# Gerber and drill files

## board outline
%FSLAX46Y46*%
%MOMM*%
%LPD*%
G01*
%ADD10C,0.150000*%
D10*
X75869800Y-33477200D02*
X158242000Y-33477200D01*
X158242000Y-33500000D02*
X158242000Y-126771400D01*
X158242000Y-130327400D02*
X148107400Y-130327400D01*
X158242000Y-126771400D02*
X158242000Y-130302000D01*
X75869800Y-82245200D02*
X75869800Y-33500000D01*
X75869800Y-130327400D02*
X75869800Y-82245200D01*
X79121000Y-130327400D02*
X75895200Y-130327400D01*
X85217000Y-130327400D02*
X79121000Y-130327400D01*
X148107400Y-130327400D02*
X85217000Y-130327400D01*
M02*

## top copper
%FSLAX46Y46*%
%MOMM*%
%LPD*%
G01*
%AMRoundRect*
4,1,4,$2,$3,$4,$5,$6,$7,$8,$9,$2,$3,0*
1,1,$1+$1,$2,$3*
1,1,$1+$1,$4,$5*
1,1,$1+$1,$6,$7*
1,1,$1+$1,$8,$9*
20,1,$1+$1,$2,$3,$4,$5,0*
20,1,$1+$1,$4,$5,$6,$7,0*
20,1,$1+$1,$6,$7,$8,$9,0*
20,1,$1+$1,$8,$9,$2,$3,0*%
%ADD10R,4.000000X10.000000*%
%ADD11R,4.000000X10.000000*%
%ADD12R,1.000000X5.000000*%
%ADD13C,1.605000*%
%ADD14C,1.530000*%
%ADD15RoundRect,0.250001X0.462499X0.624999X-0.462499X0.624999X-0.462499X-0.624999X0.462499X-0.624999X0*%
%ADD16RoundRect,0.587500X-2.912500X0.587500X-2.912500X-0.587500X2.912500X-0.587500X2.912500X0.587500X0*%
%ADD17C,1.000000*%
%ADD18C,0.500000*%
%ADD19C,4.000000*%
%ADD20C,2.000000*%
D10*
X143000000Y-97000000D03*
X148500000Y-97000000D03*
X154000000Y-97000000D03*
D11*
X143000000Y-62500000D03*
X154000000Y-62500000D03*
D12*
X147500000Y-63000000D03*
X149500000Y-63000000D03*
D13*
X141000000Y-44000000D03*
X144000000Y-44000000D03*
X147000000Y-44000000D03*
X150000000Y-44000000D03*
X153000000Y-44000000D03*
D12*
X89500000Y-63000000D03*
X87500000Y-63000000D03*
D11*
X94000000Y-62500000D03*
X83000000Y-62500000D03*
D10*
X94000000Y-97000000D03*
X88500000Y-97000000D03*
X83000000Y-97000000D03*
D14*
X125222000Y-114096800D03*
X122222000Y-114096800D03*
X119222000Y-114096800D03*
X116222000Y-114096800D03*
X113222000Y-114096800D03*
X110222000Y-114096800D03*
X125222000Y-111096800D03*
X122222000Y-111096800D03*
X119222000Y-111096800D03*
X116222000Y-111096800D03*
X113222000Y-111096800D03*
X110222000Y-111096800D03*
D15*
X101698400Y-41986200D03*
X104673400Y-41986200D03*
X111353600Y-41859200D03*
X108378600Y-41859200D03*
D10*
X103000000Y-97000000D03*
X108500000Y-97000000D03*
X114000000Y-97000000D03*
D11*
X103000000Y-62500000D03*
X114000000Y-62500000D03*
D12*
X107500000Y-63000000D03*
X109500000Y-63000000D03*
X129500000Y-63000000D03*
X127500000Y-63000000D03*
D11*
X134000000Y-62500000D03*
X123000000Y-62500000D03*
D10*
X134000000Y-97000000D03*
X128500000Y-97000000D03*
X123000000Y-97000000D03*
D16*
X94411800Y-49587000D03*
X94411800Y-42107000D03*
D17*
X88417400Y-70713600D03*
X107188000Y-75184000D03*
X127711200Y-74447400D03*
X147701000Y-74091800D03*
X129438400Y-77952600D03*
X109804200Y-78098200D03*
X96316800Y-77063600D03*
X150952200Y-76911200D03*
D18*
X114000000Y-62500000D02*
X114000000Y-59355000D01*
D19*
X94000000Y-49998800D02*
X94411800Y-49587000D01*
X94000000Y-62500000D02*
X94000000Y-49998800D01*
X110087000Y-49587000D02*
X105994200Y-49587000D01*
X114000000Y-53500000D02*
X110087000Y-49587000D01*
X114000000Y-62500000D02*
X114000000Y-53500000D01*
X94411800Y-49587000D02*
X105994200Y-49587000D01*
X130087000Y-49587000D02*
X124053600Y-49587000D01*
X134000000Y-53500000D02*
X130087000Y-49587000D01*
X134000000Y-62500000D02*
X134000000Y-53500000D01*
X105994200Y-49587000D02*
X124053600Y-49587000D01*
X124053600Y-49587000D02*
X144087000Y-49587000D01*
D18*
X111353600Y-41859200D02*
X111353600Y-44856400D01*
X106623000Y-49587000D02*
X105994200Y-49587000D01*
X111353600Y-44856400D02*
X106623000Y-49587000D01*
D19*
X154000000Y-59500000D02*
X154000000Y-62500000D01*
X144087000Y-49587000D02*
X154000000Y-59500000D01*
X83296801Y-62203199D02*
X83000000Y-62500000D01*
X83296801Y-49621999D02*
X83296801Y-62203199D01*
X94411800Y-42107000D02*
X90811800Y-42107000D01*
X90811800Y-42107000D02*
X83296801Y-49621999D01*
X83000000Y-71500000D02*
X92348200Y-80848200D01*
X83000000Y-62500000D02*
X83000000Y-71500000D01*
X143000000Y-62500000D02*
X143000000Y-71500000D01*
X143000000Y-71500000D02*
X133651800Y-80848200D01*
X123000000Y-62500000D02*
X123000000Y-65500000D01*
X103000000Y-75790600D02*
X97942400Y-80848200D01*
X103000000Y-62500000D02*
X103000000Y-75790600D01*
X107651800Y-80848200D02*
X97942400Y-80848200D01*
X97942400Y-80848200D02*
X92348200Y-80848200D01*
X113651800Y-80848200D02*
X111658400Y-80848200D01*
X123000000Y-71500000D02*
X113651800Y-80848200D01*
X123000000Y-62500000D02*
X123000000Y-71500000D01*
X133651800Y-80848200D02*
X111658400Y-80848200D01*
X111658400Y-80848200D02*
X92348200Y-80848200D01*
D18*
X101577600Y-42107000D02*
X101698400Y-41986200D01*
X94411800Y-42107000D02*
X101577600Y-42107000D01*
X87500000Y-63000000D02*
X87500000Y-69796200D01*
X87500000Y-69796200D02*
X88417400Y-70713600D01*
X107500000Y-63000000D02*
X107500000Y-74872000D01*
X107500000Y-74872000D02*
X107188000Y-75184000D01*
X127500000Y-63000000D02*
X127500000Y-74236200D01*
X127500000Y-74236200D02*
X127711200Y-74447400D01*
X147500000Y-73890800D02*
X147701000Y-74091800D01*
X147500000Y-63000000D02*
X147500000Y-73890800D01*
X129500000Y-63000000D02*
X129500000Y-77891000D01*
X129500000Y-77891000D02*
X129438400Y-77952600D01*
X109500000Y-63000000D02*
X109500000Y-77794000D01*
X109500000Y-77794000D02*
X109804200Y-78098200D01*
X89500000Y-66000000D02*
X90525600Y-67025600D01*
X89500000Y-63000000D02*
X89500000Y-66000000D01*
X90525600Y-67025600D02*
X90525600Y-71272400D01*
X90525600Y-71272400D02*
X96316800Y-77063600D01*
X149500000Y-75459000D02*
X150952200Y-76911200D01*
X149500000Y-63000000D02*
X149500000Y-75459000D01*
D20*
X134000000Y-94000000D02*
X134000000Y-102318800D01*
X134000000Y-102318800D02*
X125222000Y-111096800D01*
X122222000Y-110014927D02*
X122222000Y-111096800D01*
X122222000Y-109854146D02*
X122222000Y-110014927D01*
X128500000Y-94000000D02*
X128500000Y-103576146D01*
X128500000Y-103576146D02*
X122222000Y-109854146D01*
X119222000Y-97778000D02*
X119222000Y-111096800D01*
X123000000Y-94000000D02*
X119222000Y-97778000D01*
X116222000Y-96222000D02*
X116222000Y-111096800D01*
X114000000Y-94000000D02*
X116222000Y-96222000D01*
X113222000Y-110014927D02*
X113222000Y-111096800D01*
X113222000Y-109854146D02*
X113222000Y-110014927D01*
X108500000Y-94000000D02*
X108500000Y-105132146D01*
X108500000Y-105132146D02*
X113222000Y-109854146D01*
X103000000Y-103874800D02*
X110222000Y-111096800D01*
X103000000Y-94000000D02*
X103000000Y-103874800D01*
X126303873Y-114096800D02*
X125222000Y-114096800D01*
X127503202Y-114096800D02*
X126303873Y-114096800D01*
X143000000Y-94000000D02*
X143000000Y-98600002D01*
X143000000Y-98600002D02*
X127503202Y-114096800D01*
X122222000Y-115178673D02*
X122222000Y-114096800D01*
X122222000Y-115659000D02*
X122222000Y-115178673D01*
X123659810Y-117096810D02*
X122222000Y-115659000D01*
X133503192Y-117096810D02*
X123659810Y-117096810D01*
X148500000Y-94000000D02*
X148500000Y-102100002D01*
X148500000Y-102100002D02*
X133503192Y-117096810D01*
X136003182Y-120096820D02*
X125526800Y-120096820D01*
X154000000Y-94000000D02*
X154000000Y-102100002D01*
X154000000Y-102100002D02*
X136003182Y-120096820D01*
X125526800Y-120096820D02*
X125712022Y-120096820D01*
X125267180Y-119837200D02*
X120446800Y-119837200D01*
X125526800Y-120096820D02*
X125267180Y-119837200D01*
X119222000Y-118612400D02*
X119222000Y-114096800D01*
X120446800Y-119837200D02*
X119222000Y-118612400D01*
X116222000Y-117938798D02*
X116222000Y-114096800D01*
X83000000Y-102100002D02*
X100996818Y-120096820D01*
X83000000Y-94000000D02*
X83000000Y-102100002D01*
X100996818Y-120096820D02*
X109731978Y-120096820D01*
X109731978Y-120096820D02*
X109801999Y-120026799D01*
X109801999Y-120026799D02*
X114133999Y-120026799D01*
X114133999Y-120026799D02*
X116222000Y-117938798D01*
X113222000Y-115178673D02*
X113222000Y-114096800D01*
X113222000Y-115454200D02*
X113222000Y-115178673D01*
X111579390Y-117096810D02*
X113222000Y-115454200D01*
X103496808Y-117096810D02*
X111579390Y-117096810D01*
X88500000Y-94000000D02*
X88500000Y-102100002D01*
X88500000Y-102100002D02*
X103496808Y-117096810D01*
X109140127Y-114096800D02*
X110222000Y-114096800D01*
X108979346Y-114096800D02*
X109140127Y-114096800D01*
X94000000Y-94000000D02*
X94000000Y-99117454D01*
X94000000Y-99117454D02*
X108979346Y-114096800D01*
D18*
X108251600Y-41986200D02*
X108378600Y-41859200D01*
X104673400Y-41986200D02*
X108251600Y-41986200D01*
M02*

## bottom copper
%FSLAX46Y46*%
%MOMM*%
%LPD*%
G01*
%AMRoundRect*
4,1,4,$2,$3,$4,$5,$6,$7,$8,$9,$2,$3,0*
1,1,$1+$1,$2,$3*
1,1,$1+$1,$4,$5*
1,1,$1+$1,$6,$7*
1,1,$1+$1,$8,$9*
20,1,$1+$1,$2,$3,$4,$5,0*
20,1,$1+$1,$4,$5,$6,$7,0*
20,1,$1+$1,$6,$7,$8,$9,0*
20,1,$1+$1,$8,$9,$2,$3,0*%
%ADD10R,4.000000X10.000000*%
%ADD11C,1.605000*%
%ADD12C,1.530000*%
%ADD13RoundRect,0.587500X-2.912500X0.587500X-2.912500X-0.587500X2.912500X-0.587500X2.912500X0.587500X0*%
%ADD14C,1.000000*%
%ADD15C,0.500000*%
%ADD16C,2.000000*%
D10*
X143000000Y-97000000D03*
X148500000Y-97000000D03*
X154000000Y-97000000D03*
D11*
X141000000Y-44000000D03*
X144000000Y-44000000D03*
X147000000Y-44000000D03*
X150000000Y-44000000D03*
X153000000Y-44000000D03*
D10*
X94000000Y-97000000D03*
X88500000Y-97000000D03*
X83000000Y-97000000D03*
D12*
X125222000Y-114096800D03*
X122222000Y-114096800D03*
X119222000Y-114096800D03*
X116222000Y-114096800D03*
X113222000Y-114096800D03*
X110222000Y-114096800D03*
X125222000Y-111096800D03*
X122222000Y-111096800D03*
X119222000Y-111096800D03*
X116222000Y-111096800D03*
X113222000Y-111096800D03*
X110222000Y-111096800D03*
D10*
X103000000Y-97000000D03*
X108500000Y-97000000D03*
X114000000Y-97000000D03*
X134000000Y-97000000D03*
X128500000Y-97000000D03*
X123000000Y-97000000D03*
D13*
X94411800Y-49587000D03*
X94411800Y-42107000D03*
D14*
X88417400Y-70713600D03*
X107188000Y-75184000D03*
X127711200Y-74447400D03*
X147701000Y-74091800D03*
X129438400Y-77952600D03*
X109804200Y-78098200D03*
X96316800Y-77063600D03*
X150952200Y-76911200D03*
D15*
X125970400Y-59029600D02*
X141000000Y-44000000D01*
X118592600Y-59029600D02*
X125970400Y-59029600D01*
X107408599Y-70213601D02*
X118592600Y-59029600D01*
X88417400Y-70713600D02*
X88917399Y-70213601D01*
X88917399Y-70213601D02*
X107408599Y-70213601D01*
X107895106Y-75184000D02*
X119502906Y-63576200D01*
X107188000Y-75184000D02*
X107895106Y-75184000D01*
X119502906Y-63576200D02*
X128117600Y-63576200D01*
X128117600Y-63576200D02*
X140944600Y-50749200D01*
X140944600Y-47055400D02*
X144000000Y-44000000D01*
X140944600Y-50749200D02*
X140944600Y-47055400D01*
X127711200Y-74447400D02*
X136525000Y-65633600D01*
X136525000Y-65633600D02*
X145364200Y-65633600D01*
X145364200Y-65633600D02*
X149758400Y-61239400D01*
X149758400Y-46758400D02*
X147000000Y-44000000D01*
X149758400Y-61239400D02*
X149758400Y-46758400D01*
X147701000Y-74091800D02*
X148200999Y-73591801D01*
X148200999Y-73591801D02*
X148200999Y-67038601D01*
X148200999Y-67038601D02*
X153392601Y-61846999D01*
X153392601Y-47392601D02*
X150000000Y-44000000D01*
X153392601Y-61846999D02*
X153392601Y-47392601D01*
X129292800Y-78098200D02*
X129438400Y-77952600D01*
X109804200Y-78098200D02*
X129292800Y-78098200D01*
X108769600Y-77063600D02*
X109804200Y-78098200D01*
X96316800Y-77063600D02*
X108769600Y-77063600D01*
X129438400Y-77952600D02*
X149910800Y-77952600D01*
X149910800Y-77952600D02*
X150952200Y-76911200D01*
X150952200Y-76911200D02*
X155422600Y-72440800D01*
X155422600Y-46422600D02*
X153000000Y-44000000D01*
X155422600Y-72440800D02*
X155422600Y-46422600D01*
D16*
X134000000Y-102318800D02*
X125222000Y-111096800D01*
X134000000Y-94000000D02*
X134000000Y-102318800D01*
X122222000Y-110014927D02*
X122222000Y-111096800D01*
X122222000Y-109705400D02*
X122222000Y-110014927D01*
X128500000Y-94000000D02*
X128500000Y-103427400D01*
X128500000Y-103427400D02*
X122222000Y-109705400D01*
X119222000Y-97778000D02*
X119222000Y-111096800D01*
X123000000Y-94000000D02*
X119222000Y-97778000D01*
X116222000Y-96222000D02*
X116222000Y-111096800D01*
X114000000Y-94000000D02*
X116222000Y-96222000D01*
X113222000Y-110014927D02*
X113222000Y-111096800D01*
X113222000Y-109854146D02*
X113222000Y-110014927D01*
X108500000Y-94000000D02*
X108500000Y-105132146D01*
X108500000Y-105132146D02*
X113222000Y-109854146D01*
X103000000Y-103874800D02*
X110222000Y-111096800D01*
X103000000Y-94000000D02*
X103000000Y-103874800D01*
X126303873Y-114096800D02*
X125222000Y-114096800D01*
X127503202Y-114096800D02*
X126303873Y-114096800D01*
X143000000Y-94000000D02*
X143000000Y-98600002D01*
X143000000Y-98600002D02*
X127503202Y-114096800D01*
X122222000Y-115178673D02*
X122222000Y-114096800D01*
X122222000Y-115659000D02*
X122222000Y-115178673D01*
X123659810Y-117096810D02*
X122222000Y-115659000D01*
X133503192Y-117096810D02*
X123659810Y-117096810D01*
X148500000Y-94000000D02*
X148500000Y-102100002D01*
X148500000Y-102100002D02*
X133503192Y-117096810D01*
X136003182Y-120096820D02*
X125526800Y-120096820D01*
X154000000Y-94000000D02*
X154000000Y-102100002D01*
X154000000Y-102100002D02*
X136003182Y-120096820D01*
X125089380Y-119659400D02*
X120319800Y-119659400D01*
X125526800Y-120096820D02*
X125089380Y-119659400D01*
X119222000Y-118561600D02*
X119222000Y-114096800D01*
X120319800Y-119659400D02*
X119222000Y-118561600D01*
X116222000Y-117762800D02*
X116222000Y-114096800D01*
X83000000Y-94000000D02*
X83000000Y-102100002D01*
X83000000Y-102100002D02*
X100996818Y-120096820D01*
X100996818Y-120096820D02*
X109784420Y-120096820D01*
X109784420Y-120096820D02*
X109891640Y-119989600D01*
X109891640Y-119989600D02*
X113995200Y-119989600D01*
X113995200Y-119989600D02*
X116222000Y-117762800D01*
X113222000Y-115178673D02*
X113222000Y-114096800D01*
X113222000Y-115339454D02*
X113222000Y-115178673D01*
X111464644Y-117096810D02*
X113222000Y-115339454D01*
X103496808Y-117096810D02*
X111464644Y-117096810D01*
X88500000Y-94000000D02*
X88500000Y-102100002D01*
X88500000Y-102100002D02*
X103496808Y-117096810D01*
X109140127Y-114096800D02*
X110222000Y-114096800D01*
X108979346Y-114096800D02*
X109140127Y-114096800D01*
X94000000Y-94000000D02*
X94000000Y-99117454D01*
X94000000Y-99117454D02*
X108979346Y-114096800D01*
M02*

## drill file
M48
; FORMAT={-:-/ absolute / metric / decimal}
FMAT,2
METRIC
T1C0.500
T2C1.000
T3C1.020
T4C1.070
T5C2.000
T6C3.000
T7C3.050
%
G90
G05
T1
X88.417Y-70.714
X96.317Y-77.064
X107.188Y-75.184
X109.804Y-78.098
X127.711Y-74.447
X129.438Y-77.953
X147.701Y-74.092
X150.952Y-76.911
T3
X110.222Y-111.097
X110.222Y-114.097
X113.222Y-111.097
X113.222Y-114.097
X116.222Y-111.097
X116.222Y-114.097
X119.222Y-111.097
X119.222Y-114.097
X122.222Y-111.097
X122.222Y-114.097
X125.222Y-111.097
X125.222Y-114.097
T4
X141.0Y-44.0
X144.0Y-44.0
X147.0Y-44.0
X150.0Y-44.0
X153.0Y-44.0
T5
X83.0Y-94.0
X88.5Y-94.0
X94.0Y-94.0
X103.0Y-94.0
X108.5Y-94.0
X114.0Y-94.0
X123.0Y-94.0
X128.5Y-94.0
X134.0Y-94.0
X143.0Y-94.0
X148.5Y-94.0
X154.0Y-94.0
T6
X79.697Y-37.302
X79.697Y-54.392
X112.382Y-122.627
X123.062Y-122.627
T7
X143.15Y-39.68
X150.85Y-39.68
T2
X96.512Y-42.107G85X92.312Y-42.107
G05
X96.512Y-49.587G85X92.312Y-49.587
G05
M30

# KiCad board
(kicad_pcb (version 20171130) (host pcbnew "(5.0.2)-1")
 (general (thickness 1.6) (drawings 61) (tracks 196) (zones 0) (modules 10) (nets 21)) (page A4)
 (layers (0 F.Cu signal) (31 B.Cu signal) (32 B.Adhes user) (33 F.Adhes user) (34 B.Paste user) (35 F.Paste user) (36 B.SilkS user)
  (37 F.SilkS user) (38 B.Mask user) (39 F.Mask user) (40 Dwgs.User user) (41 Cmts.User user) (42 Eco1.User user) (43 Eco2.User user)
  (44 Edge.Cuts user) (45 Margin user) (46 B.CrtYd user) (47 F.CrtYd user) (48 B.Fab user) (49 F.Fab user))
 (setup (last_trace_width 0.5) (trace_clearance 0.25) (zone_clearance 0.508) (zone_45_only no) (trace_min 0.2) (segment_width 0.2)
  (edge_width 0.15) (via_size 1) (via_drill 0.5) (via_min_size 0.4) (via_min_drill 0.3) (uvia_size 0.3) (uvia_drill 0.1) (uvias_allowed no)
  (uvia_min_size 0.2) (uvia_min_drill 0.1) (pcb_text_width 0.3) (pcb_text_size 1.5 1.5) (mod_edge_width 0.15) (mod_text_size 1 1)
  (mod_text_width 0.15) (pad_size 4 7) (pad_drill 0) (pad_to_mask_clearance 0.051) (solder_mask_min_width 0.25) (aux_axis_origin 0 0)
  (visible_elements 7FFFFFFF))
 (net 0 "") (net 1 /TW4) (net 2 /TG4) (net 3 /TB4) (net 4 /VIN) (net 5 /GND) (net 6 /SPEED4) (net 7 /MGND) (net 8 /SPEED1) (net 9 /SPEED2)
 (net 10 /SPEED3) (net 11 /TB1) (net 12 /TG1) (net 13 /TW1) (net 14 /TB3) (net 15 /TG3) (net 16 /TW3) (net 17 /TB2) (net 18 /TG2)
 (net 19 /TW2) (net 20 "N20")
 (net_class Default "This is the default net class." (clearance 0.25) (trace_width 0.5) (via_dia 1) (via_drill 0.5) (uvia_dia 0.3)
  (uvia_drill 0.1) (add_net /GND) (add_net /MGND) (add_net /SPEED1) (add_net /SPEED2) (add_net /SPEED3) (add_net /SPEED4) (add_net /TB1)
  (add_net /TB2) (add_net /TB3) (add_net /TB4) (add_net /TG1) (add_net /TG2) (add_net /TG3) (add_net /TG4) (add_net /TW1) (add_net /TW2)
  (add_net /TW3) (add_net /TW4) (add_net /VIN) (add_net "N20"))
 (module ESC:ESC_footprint (layer F.Cu) (at 140 95)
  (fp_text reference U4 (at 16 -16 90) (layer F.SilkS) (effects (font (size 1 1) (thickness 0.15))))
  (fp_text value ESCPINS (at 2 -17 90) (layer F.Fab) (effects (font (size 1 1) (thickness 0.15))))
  (pad 3 thru_hole rect (at 3 -1) (size 4 10) (drill 2 (offset 0 3)) (layers *.Cu *.Mask) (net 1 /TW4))
  (pad 2 thru_hole rect (at 8.5 -1) (size 4 10) (drill 2 (offset 0 3)) (layers *.Cu *.Mask) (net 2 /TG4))
  (pad 1 thru_hole rect (at 14 -1) (size 4 10) (drill 2 (offset 0 3)) (layers *.Cu *.Mask) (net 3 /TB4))
  (pad 6 smd rect (at 3 -32.5) (size 4 10) (layers F.Cu F.Paste F.Mask) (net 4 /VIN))
  (pad 7 smd rect (at 14 -32.5) (size 4 10) (layers F.Cu F.Paste F.Mask) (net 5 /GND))
  (pad 4 smd rect (at 7.5 -32) (size 1 5) (layers F.Cu F.Paste F.Mask) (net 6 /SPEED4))
  (pad 5 smd rect (at 9.5 -32) (size 1 5) (layers F.Cu F.Paste F.Mask) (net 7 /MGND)))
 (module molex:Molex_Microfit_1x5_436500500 (layer F.Cu) (at 141 44 180)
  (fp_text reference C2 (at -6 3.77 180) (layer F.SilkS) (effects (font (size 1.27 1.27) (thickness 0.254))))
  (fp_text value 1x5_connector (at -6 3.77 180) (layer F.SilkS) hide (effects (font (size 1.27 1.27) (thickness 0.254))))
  (pad 1 thru_hole circle (at 0 0 180) (size 1.605 1.605) (drill 1.07) (layers *.Cu *.Mask) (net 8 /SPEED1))
  (pad 2 thru_hole circle (at -3 0 180) (size 1.605 1.605) (drill 1.07) (layers *.Cu *.Mask) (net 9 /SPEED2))
  (pad 3 thru_hole circle (at -6 0 180) (size 1.605 1.605) (drill 1.07) (layers *.Cu *.Mask) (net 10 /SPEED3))
  (pad 4 thru_hole circle (at -9 0 180) (size 1.605 1.605) (drill 1.07) (layers *.Cu *.Mask) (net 6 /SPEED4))
  (pad 5 thru_hole circle (at -12 0 180) (size 1.605 1.605) (drill 1.07) (layers *.Cu *.Mask) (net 7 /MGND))
  (pad MH1 np_thru_hole circle (at -2.15 4.32 180) (size 3.05 0) (drill 3.05) (layers *.Cu *.Mask))
  (pad MH2 np_thru_hole circle (at -9.85 4.32 180) (size 3.05 0) (drill 3.05) (layers *.Cu *.Mask)))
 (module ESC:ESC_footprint (layer F.Cu) (at 80 95)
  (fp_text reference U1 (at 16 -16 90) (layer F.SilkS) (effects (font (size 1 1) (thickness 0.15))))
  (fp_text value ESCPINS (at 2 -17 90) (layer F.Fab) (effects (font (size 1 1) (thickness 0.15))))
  (pad 5 smd rect (at 9.5 -32) (size 1 5) (layers F.Cu F.Paste F.Mask) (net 7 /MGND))
  (pad 4 smd rect (at 7.5 -32) (size 1 5) (layers F.Cu F.Paste F.Mask) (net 8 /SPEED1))
  (pad 7 smd rect (at 14 -32.5) (size 4 10) (layers F.Cu F.Paste F.Mask) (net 5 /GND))
  (pad 6 smd rect (at 3 -32.5) (size 4 10) (layers F.Cu F.Paste F.Mask) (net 4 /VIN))
  (pad 1 thru_hole rect (at 14 -1) (size 4 10) (drill 2 (offset 0 3)) (layers *.Cu *.Mask) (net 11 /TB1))
  (pad 2 thru_hole rect (at 8.5 -1) (size 4 10) (drill 2 (offset 0 3)) (layers *.Cu *.Mask) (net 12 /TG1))
  (pad 3 thru_hole rect (at 3 -1) (size 4 10) (drill 2 (offset 0 3)) (layers *.Cu *.Mask) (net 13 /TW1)))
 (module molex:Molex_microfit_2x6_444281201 (layer F.Cu) (at 125.222 114.0968)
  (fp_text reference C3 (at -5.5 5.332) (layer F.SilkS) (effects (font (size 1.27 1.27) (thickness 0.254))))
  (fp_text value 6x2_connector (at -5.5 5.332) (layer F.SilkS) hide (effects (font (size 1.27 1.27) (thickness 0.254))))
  (pad 1 thru_hole circle (at 0 0) (size 1.53 1.53) (drill 1.02) (layers *.Cu *.Mask) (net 1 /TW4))
  (pad 2 thru_hole circle (at -3 0) (size 1.53 1.53) (drill 1.02) (layers *.Cu *.Mask) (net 2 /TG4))
  (pad 3 thru_hole circle (at -6 0) (size 1.53 1.53) (drill 1.02) (layers *.Cu *.Mask) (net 3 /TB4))
  (pad 4 thru_hole circle (at -9 0) (size 1.53 1.53) (drill 1.02) (layers *.Cu *.Mask) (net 13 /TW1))
  (pad 5 thru_hole circle (at -12 0) (size 1.53 1.53) (drill 1.02) (layers *.Cu *.Mask) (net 12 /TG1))
  (pad 6 thru_hole circle (at -15 0) (size 1.53 1.53) (drill 1.02) (layers *.Cu *.Mask) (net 11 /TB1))
  (pad 7 thru_hole circle (at 0 -3) (size 1.53 1.53) (drill 1.02) (layers *.Cu *.Mask) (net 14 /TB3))
  (pad 8 thru_hole circle (at -3 -3) (size 1.53 1.53) (drill 1.02) (layers *.Cu *.Mask) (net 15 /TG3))
  (pad 9 thru_hole circle (at -6 -3) (size 1.53 1.53) (drill 1.02) (layers *.Cu *.Mask) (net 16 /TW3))
  (pad 10 thru_hole circle (at -9 -3) (size 1.53 1.53) (drill 1.02) (layers *.Cu *.Mask) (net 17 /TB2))
  (pad 11 thru_hole circle (at -12 -3) (size 1.53 1.53) (drill 1.02) (layers *.Cu *.Mask) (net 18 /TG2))
  (pad 12 thru_hole circle (at -15 -3) (size 1.53 1.53) (drill 1.02) (layers *.Cu *.Mask) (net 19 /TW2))
  (pad MH1 np_thru_hole circle (at -12.84 8.53) (size 3 0) (drill 3) (layers *.Cu *.Mask))
  (pad MH2 np_thru_hole circle (at -2.16 8.53) (size 3 0) (drill 3) (layers *.Cu *.Mask)))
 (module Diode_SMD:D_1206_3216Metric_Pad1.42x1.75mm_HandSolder (layer F.Cu) (at 103.1859 41.9862 180)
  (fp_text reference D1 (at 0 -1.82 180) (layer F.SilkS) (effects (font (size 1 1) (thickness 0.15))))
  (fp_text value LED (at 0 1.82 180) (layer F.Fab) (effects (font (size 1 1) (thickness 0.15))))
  (pad 2 smd roundrect (at 1.4875 0 180) (size 1.425 1.75) (layers F.Cu F.Paste F.Mask) (roundrect_rratio 0.175439) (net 4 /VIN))
  (pad 1 smd roundrect (at -1.4875 0 180) (size 1.425 1.75) (layers F.Cu F.Paste F.Mask) (roundrect_rratio 0.175439) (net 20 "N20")))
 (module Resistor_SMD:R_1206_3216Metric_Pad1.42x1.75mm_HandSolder (layer F.Cu) (at 109.8661 41.8592 180)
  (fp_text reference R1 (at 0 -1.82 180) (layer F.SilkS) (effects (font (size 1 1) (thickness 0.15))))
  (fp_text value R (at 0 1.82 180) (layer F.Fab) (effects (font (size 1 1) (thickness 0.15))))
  (pad 1 smd roundrect (at -1.4875 0 180) (size 1.425 1.75) (layers F.Cu F.Paste F.Mask) (roundrect_rratio 0.175439) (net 5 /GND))
  (pad 2 smd roundrect (at 1.4875 0 180) (size 1.425 1.75) (layers F.Cu F.Paste F.Mask) (roundrect_rratio 0.175439) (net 20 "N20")))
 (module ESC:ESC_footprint (layer F.Cu) (at 100 95)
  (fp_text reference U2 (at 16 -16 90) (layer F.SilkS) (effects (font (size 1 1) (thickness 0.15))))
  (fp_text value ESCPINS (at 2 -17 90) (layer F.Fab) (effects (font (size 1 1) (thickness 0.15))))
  (pad 3 thru_hole rect (at 3 -1) (size 4 10) (drill 2 (offset 0 3)) (layers *.Cu *.Mask) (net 19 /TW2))
  (pad 2 thru_hole rect (at 8.5 -1) (size 4 10) (drill 2 (offset 0 3)) (layers *.Cu *.Mask) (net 18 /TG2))
  (pad 1 thru_hole rect (at 14 -1) (size 4 10) (drill 2 (offset 0 3)) (layers *.Cu *.Mask) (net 17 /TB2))
  (pad 6 smd rect (at 3 -32.5) (size 4 10) (layers F.Cu F.Paste F.Mask) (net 4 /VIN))
  (pad 7 smd rect (at 14 -32.5) (size 4 10) (layers F.Cu F.Paste F.Mask) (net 5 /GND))
  (pad 4 smd rect (at 7.5 -32) (size 1 5) (layers F.Cu F.Paste F.Mask) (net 9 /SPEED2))
  (pad 5 smd rect (at 9.5 -32) (size 1 5) (layers F.Cu F.Paste F.Mask) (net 7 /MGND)))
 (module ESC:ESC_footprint (layer F.Cu) (at 120 95)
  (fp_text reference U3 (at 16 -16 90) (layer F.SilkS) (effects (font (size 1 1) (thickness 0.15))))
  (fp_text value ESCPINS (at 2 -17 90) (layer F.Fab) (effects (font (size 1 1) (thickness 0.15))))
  (pad 5 smd rect (at 9.5 -32) (size 1 5) (layers F.Cu F.Paste F.Mask) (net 7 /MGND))
  (pad 4 smd rect (at 7.5 -32) (size 1 5) (layers F.Cu F.Paste F.Mask) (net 10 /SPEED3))
  (pad 7 smd rect (at 14 -32.5) (size 4 10) (layers F.Cu F.Paste F.Mask) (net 5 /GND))
  (pad 6 smd rect (at 3 -32.5) (size 4 10) (layers F.Cu F.Paste F.Mask) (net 4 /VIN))
  (pad 1 thru_hole rect (at 14 -1) (size 4 10) (drill 2 (offset 0 3)) (layers *.Cu *.Mask) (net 14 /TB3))
  (pad 2 thru_hole rect (at 8.5 -1) (size 4 10) (drill 2 (offset 0 3)) (layers *.Cu *.Mask) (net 15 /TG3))
  (pad 3 thru_hole rect (at 3 -1) (size 4 10) (drill 2 (offset 0 3)) (layers *.Cu *.Mask) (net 16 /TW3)))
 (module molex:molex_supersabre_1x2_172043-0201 (layer F.Cu) (at 94.4118 45.847 270)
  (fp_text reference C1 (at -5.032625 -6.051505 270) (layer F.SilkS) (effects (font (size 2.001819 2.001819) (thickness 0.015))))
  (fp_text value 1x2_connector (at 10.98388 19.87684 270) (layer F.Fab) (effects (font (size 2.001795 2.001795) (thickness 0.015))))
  (pad 2 thru_hole roundrect (at 3.74 0 270) (size 2.35 7) (drill oval 1 5.2) (layers *.Cu *.Mask) (roundrect_rratio 0.25) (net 5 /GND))
  (pad 1 thru_hole roundrect (at -3.74 0 270) (size 2.35 7) (drill oval 1 5.2) (layers *.Cu *.Mask) (roundrect_rratio 0.25) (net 4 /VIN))
  (pad None np_thru_hole circle (at -8.545 14.715 270) (size 3 3) (drill 3) (layers *.Cu *.Mask))
  (pad None np_thru_hole circle (at 8.545 14.715 270) (size 3 3) (drill 3) (layers *.Cu *.Mask)))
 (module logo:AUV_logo (layer F.Cu) (at 87.5 125)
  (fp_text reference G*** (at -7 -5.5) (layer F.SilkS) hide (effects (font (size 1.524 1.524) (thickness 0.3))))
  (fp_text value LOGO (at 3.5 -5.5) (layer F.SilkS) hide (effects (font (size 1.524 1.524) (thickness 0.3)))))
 (gr_line (start 75.8698 33.4772) (end 158.242 33.4772) (layer Edge.Cuts) (width 0.15))
 (gr_line (start 158.242 33.5) (end 158.242 126.7714) (layer Edge.Cuts) (width 0.15))
 (gr_line (start 158.242 130.3274) (end 148.1074 130.3274) (layer Edge.Cuts) (width 0.15))
 (gr_line (start 158.242 126.7714) (end 158.242 130.302) (layer Edge.Cuts) (width 0.15))
 (gr_line (start 75.8698 82.2452) (end 75.8698 33.5) (layer Edge.Cuts) (width 0.15))
 (gr_line (start 75.8698 130.3274) (end 75.8698 82.2452) (layer Edge.Cuts) (width 0.15))
 (gr_line (start 79.121 130.3274) (end 75.8952 130.3274) (layer Edge.Cuts) (width 0.15))
 (gr_line (start 85.217 130.3274) (end 79.121 130.3274) (layer Edge.Cuts) (width 0.15))
 (gr_line (start 148.1074 130.3274) (end 85.217 130.3274) (layer Edge.Cuts) (width 0.15))
 (segment (start 114 62.5) (end 114 59.355) (width 0.5) (layer F.Cu) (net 5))
 (segment (start 94 49.9988) (end 94.4118 49.587) (width 4) (layer F.Cu) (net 5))
 (segment (start 94 62.5) (end 94 49.9988) (width 4) (layer F.Cu) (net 5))
 (segment (start 110.087 49.587) (end 105.9942 49.587) (width 4) (layer F.Cu) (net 5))
 (segment (start 114 53.5) (end 110.087 49.587) (width 4) (layer F.Cu) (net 5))
 (segment (start 114 62.5) (end 114 53.5) (width 4) (layer F.Cu) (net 5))
 (segment (start 94.4118 49.587) (end 105.9942 49.587) (width 4) (layer F.Cu) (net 5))
 (segment (start 130.087 49.587) (end 124.0536 49.587) (width 4) (layer F.Cu) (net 5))
 (segment (start 134 53.5) (end 130.087 49.587) (width 4) (layer F.Cu) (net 5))
 (segment (start 134 62.5) (end 134 53.5) (width 4) (layer F.Cu) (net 5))
 (segment (start 105.9942 49.587) (end 124.0536 49.587) (width 4) (layer F.Cu) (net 5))
 (segment (start 124.0536 49.587) (end 144.087 49.587) (width 4) (layer F.Cu) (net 5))
 (segment (start 111.3536 41.8592) (end 111.3536 44.8564) (width 0.5) (layer F.Cu) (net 5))
 (segment (start 106.623 49.587) (end 105.9942 49.587) (width 0.5) (layer F.Cu) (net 5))
 (segment (start 111.3536 44.8564) (end 106.623 49.587) (width 0.5) (layer F.Cu) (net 5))
 (segment (start 154 59.5) (end 154 62.5) (width 4) (layer F.Cu) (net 5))
 (segment (start 144.087 49.587) (end 154 59.5) (width 4) (layer F.Cu) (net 5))
 (segment (start 83.296801 62.203199) (end 83 62.5) (width 4) (layer F.Cu) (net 4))
 (segment (start 83.296801 49.621999) (end 83.296801 62.203199) (width 4) (layer F.Cu) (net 4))
 (segment (start 94.4118 42.107) (end 90.8118 42.107) (width 4) (layer F.Cu) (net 4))
 (segment (start 90.8118 42.107) (end 83.296801 49.621999) (width 4) (layer F.Cu) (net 4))
 (segment (start 83 71.5) (end 92.3482 80.8482) (width 4) (layer F.Cu) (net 4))
 (segment (start 83 62.5) (end 83 71.5) (width 4) (layer F.Cu) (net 4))
 (segment (start 143 62.5) (end 143 71.5) (width 4) (layer F.Cu) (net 4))
 (segment (start 143 71.5) (end 133.6518 80.8482) (width 4) (layer F.Cu) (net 4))
 (segment (start 123 62.5) (end 123 65.5) (width 4) (layer F.Cu) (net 4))
 (segment (start 103 75.7906) (end 97.9424 80.8482) (width 4) (layer F.Cu) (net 4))
 (segment (start 103 62.5) (end 103 75.7906) (width 4) (layer F.Cu) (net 4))
 (segment (start 107.6518 80.8482) (end 97.9424 80.8482) (width 4) (layer F.Cu) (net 4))
 (segment (start 97.9424 80.8482) (end 92.3482 80.8482) (width 4) (layer F.Cu) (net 4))
 (segment (start 113.6518 80.8482) (end 111.6584 80.8482) (width 4) (layer F.Cu) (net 4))
 (segment (start 123 71.5) (end 113.6518 80.8482) (width 4) (layer F.Cu) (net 4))
 (segment (start 123 62.5) (end 123 71.5) (width 4) (layer F.Cu) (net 4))
 (segment (start 133.6518 80.8482) (end 111.6584 80.8482) (width 4) (layer F.Cu) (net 4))
 (segment (start 111.6584 80.8482) (end 92.3482 80.8482) (width 4) (layer F.Cu) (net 4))
 (segment (start 101.5776 42.107) (end 101.6984 41.9862) (width 0.5) (layer F.Cu) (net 4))
 (segment (start 94.4118 42.107) (end 101.5776 42.107) (width 0.5) (layer F.Cu) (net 4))
 (via (at 88.4174 70.7136) (size 1) (drill 0.5) (layers F.Cu B.Cu) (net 8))
 (segment (start 87.5 63) (end 87.5 69.7962) (width 0.5) (layer F.Cu) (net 8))
 (segment (start 87.5 69.7962) (end 88.4174 70.7136) (width 0.5) (layer F.Cu) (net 8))
 (segment (start 125.9704 59.0296) (end 141 44) (width 0.5) (layer B.Cu) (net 8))
 (segment (start 118.5926 59.0296) (end 125.9704 59.0296) (width 0.5) (layer B.Cu) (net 8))
 (segment (start 107.408599 70.213601) (end 118.5926 59.0296) (width 0.5) (layer B.Cu) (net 8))
 (segment (start 88.4174 70.7136) (end 88.917399 70.213601) (width 0.5) (layer B.Cu) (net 8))
 (segment (start 88.917399 70.213601) (end 107.408599 70.213601) (width 0.5) (layer B.Cu) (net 8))
 (via (at 107.188 75.184) (size 1) (drill 0.5) (layers F.Cu B.Cu) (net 9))
 (segment (start 107.5 63) (end 107.5 74.872) (width 0.5) (layer F.Cu) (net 9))
 (segment (start 107.5 74.872) (end 107.188 75.184) (width 0.5) (layer F.Cu) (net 9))
 (segment (start 107.895106 75.184) (end 119.502906 63.5762) (width 0.5) (layer B.Cu) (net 9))
 (segment (start 107.188 75.184) (end 107.895106 75.184) (width 0.5) (layer B.Cu) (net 9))
 (segment (start 119.502906 63.5762) (end 128.1176 63.5762) (width 0.5) (layer B.Cu) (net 9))
 (segment (start 128.1176 63.5762) (end 140.9446 50.7492) (width 0.5) (layer B.Cu) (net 9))
 (segment (start 140.9446 47.0554) (end 144 44) (width 0.5) (layer B.Cu) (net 9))
 (segment (start 140.9446 50.7492) (end 140.9446 47.0554) (width 0.5) (layer B.Cu) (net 9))
 (via (at 127.7112 74.4474) (size 1) (drill 0.5) (layers F.Cu B.Cu) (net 10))
 (segment (start 127.5 63) (end 127.5 74.2362) (width 0.5) (layer F.Cu) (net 10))
 (segment (start 127.5 74.2362) (end 127.7112 74.4474) (width 0.5) (layer F.Cu) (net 10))
 (segment (start 127.7112 74.4474) (end 136.525 65.6336) (width 0.5) (layer B.Cu) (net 10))
 (segment (start 136.525 65.6336) (end 145.3642 65.6336) (width 0.5) (layer B.Cu) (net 10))
 (segment (start 145.3642 65.6336) (end 149.7584 61.2394) (width 0.5) (layer B.Cu) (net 10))
 (segment (start 149.7584 46.7584) (end 147 44) (width 0.5) (layer B.Cu) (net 10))
 (segment (start 149.7584 61.2394) (end 149.7584 46.7584) (width 0.5) (layer B.Cu) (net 10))
 (segment (start 147.5 73.8908) (end 147.701 74.0918) (width 0.5) (layer F.Cu) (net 6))
 (segment (start 147.5 63) (end 147.5 73.8908) (width 0.5) (layer F.Cu) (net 6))
 (segment (start 147.701 74.0918) (end 148.200999 73.591801) (width 0.5) (layer B.Cu) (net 6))
 (segment (start 148.200999 73.591801) (end 148.200999 67.038601) (width 0.5) (layer B.Cu) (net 6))
 (segment (start 148.200999 67.038601) (end 153.392601 61.846999) (width 0.5) (layer B.Cu) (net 6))
 (via (at 147.701 74.0918) (size 1) (drill 0.5) (layers F.Cu B.Cu) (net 6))
 (segment (start 153.392601 47.392601) (end 150 44) (width 0.5) (layer B.Cu) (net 6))
 (segment (start 153.392601 61.846999) (end 153.392601 47.392601) (width 0.5) (layer B.Cu) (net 6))
 (via (at 129.4384 77.9526) (size 1) (drill 0.5) (layers F.Cu B.Cu) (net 7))
 (segment (start 129.5 63) (end 129.5 77.891) (width 0.5) (layer F.Cu) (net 7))
 (segment (start 129.5 77.891) (end 129.4384 77.9526) (width 0.5) (layer F.Cu) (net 7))
 (via (at 109.8042 78.0982) (size 1) (drill 0.5) (layers F.Cu B.Cu) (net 7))
 (segment (start 109.5 63) (end 109.5 77.794) (width 0.5) (layer F.Cu) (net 7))
 (segment (start 109.5 77.794) (end 109.8042 78.0982) (width 0.5) (layer F.Cu) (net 7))
 (segment (start 89.5 66) (end 90.5256 67.0256) (width 0.5) (layer F.Cu) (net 7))
 (segment (start 89.5 63) (end 89.5 66) (width 0.5) (layer F.Cu) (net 7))
 (via (at 96.3168 77.0636) (size 1) (drill 0.5) (layers F.Cu B.Cu) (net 7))
 (segment (start 90.5256 67.0256) (end 90.5256 71.2724) (width 0.5) (layer F.Cu) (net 7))
 (segment (start 90.5256 71.2724) (end 96.3168 77.0636) (width 0.5) (layer F.Cu) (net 7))
 (segment (start 129.2928 78.0982) (end 129.4384 77.9526) (width 0.5) (layer B.Cu) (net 7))
 (segment (start 109.8042 78.0982) (end 129.2928 78.0982) (width 0.5) (layer B.Cu) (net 7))
 (segment (start 108.7696 77.0636) (end 109.8042 78.0982) (width 0.5) (layer B.Cu) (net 7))
 (segment (start 96.3168 77.0636) (end 108.7696 77.0636) (width 0.5) (layer B.Cu) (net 7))
 (segment (start 129.4384 77.9526) (end 149.9108 77.9526) (width 0.5) (layer B.Cu) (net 7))
 (segment (start 149.9108 77.9526) (end 150.9522 76.9112) (width 0.5) (layer B.Cu) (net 7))
 (segment (start 149.5 75.459) (end 150.9522 76.9112) (width 0.5) (layer F.Cu) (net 7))
 (segment (start 150.9522 76.9112) (end 155.4226 72.4408) (width 0.5) (layer B.Cu) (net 7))
 (segment (start 149.5 63) (end 149.5 75.459) (width 0.5) (layer F.Cu) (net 7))
 (via (at 150.9522 76.9112) (size 1) (drill 0.5) (layers F.Cu B.Cu) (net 7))
 (segment (start 155.4226 46.4226) (end 153 44) (width 0.5) (layer B.Cu) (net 7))
 (segment (start 155.4226 72.4408) (end 155.4226 46.4226) (width 0.5) (layer B.Cu) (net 7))
 (segment (start 134 94) (end 134 102.3188) (width 2) (layer F.Cu) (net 14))
 (segment (start 134 102.3188) (end 125.222 111.0968) (width 2) (layer F.Cu) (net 14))
 (segment (start 134 102.3188) (end 125.222 111.0968) (width 2) (layer B.Cu) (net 14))
 (segment (start 134 94) (end 134 102.3188) (width 2) (layer B.Cu) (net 14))
 (segment (start 122.222 110.014927) (end 122.222 111.0968) (width 2) (layer B.Cu) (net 15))
 (segment (start 122.222 109.7054) (end 122.222 110.014927) (width 2) (layer B.Cu) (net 15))
 (segment (start 128.5 94) (end 128.5 103.4274) (width 2) (layer B.Cu) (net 15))
 (segment (start 128.5 103.4274) (end 122.222 109.7054) (width 2) (layer B.Cu) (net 15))
 (segment (start 122.222 110.014927) (end 122.222 111.0968) (width 2) (layer F.Cu) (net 15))
 (segment (start 122.222 109.854146) (end 122.222 110.014927) (width 2) (layer F.Cu) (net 15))
 (segment (start 128.5 94) (end 128.5 103.576146) (width 2) (layer F.Cu) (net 15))
 (segment (start 128.5 103.576146) (end 122.222 109.854146) (width 2) (layer F.Cu) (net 15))
 (segment (start 119.222 97.778) (end 119.222 111.0968) (width 2) (layer F.Cu) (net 16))
 (segment (start 123 94) (end 119.222 97.778) (width 2) (layer F.Cu) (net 16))
 (segment (start 119.222 97.778) (end 119.222 111.0968) (width 2) (layer B.Cu) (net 16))
 (segment (start 123 94) (end 119.222 97.778) (width 2) (layer B.Cu) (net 16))
 (segment (start 116.222 96.222) (end 116.222 111.0968) (width 2) (layer F.Cu) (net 17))
 (segment (start 114 94) (end 116.222 96.222) (width 2) (layer F.Cu) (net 17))
 (segment (start 116.222 96.222) (end 116.222 111.0968) (width 2) (layer B.Cu) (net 17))
 (segment (start 114 94) (end 116.222 96.222) (width 2) (layer B.Cu) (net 17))
 (segment (start 113.222 110.014927) (end 113.222 111.0968) (width 2) (layer B.Cu) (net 18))
 (segment (start 113.222 109.854146) (end 113.222 110.014927) (width 2) (layer B.Cu) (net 18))
 (segment (start 108.5 94) (end 108.5 105.132146) (width 2) (layer B.Cu) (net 18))
 (segment (start 108.5 105.132146) (end 113.222 109.854146) (width 2) (layer B.Cu) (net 18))
 (segment (start 113.222 110.014927) (end 113.222 111.0968) (width 2) (layer F.Cu) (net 18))
 (segment (start 113.222 109.854146) (end 113.222 110.014927) (width 2) (layer F.Cu) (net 18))
 (segment (start 108.5 94) (end 108.5 105.132146) (width 2) (layer F.Cu) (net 18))
 (segment (start 108.5 105.132146) (end 113.222 109.854146) (width 2) (layer F.Cu) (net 18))
 (segment (start 103 103.8748) (end 110.222 111.0968) (width 2) (layer F.Cu) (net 19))
 (segment (start 103 94) (end 103 103.8748) (width 2) (layer F.Cu) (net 19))
 (segment (start 103 103.8748) (end 110.222 111.0968) (width 2) (layer B.Cu) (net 19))
 (segment (start 103 94) (end 103 103.8748) (width 2) (layer B.Cu) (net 19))
 (segment (start 126.303873 114.0968) (end 125.222 114.0968) (width 2) (layer F.Cu) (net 1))
 (segment (start 127.503202 114.0968) (end 126.303873 114.0968) (width 2) (layer F.Cu) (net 1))
 (segment (start 143 94) (end 143 98.600002) (width 2) (layer F.Cu) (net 1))
 (segment (start 143 98.600002) (end 127.503202 114.0968) (width 2) (layer F.Cu) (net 1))
 (segment (start 126.303873 114.0968) (end 125.222 114.0968) (width 2) (layer B.Cu) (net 1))
 (segment (start 127.503202 114.0968) (end 126.303873 114.0968) (width 2) (layer B.Cu) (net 1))
 (segment (start 143 94) (end 143 98.600002) (width 2) (layer B.Cu) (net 1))
 (segment (start 143 98.600002) (end 127.503202 114.0968) (width 2) (layer B.Cu) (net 1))
 (segment (start 122.222 115.178673) (end 122.222 114.0968) (width 2) (layer F.Cu) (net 2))
 (segment (start 122.222 115.659) (end 122.222 115.178673) (width 2) (layer F.Cu) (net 2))
 (segment (start 123.65981 117.09681) (end 122.222 115.659) (width 2) (layer F.Cu) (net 2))
 (segment (start 133.503192 117.09681) (end 123.65981 117.09681) (width 2) (layer F.Cu) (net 2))
 (segment (start 148.5 94) (end 148.5 102.100002) (width 2) (layer F.Cu) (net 2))
 (segment (start 148.5 102.100002) (end 133.503192 117.09681) (width 2) (layer F.Cu) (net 2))
 (segment (start 122.222 115.178673) (end 122.222 114.0968) (width 2) (layer B.Cu) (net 2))
 (segment (start 122.222 115.659) (end 122.222 115.178673) (width 2) (layer B.Cu) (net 2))
 (segment (start 123.65981 117.09681) (end 122.222 115.659) (width 2) (layer B.Cu) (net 2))
 (segment (start 133.503192 117.09681) (end 123.65981 117.09681) (width 2) (layer B.Cu) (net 2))
 (segment (start 148.5 94) (end 148.5 102.100002) (width 2) (layer B.Cu) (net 2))
 (segment (start 148.5 102.100002) (end 133.503192 117.09681) (width 2) (layer B.Cu) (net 2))
 (segment (start 136.003182 120.09682) (end 125.5268 120.09682) (width 2) (layer F.Cu) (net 3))
 (segment (start 154 94) (end 154 102.100002) (width 2) (layer F.Cu) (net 3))
 (segment (start 154 102.100002) (end 136.003182 120.09682) (width 2) (layer F.Cu) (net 3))
 (segment (start 125.5268 120.09682) (end 125.712022 120.09682) (width 2) (layer F.Cu) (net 3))
 (segment (start 125.26718 119.8372) (end 120.4468 119.8372) (width 2) (layer F.Cu) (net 3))
 (segment (start 125.5268 120.09682) (end 125.26718 119.8372) (width 2) (layer F.Cu) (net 3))
 (segment (start 119.222 118.6124) (end 119.222 114.0968) (width 2) (layer F.Cu) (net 3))
 (segment (start 120.4468 119.8372) (end 119.222 118.6124) (width 2) (layer F.Cu) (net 3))
 (segment (start 136.003182 120.09682) (end 125.5268 120.09682) (width 2) (layer B.Cu) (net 3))
 (segment (start 154 94) (end 154 102.100002) (width 2) (layer B.Cu) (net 3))
 (segment (start 154 102.100002) (end 136.003182 120.09682) (width 2) (layer B.Cu) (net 3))
 (segment (start 125.08938 119.6594) (end 120.3198 119.6594) (width 2) (layer B.Cu) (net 3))
 (segment (start 125.5268 120.09682) (end 125.08938 119.6594) (width 2) (layer B.Cu) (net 3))
 (segment (start 119.222 118.5616) (end 119.222 114.0968) (width 2) (layer B.Cu) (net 3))
 (segment (start 120.3198 119.6594) (end 119.222 118.5616) (width 2) (layer B.Cu) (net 3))
 (segment (start 116.222 117.938798) (end 116.222 114.0968) (width 2) (layer F.Cu) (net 13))
 (segment (start 83 102.100002) (end 100.996818 120.09682) (width 2) (layer F.Cu) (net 13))
 (segment (start 83 94) (end 83 102.100002) (width 2) (layer F.Cu) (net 13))
 (segment (start 100.996818 120.09682) (end 109.731978 120.09682) (width 2) (layer F.Cu) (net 13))
 (segment (start 109.731978 120.09682) (end 109.801999 120.026799) (width 2) (layer F.Cu) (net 13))
 (segment (start 109.801999 120.026799) (end 114.133999 120.026799) (width 2) (layer F.Cu) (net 13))
 (segment (start 114.133999 120.026799) (end 116.222 117.938798) (width 2) (layer F.Cu) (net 13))
 (segment (start 116.222 117.7628) (end 116.222 114.0968) (width 2) (layer B.Cu) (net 13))
 (segment (start 83 94) (end 83 102.100002) (width 2) (layer B.Cu) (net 13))
 (segment (start 83 102.100002) (end 100.996818 120.09682) (width 2) (layer B.Cu) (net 13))
 (segment (start 100.996818 120.09682) (end 109.78442 120.09682) (width 2) (layer B.Cu) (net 13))
 (segment (start 109.78442 120.09682) (end 109.89164 119.9896) (width 2) (layer B.Cu) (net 13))
 (segment (start 109.89164 119.9896) (end 113.9952 119.9896) (width 2) (layer B.Cu) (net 13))
 (segment (start 113.9952 119.9896) (end 116.222 117.7628) (width 2) (layer B.Cu) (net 13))
 (segment (start 113.222 115.178673) (end 113.222 114.0968) (width 2) (layer F.Cu) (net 12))
 (segment (start 113.222 115.4542) (end 113.222 115.178673) (width 2) (layer F.Cu) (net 12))
 (segment (start 111.57939 117.09681) (end 113.222 115.4542) (width 2) (layer F.Cu) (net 12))
 (segment (start 103.496808 117.09681) (end 111.57939 117.09681) (width 2) (layer F.Cu) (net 12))
 (segment (start 88.5 94) (end 88.5 102.100002) (width 2) (layer F.Cu) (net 12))
 (segment (start 88.5 102.100002) (end 103.496808 117.09681) (width 2) (layer F.Cu) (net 12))
 (segment (start 113.222 115.178673) (end 113.222 114.0968) (width 2) (layer B.Cu) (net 12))
 (segment (start 113.222 115.339454) (end 113.222 115.178673) (width 2) (layer B.Cu) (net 12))
 (segment (start 111.464644 117.09681) (end 113.222 115.339454) (width 2) (layer B.Cu) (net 12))
 (segment (start 103.496808 117.09681) (end 111.464644 117.09681) (width 2) (layer B.Cu) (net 12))
 (segment (start 88.5 94) (end 88.5 102.100002) (width 2) (layer B.Cu) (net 12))
 (segment (start 88.5 102.100002) (end 103.496808 117.09681) (width 2) (layer B.Cu) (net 12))
 (segment (start 109.140127 114.0968) (end 110.222 114.0968) (width 2) (layer F.Cu) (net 11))
 (segment (start 108.979346 114.0968) (end 109.140127 114.0968) (width 2) (layer F.Cu) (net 11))
 (segment (start 94 94) (end 94 99.117454) (width 2) (layer F.Cu) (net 11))
 (segment (start 94 99.117454) (end 108.979346 114.0968) (width 2) (layer F.Cu) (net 11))
 (segment (start 109.140127 114.0968) (end 110.222 114.0968) (width 2) (layer B.Cu) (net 11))
 (segment (start 108.979346 114.0968) (end 109.140127 114.0968) (width 2) (layer B.Cu) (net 11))
 (segment (start 94 94) (end 94 99.117454) (width 2) (layer B.Cu) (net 11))
 (segment (start 94 99.117454) (end 108.979346 114.0968) (width 2) (layer B.Cu) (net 11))
 (segment (start 108.2516 41.9862) (end 108.3786 41.8592) (width 0.5) (layer F.Cu) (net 20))
 (segment (start 104.6734 41.9862) (end 108.2516 41.9862) (width 0.5) (layer F.Cu) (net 20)))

